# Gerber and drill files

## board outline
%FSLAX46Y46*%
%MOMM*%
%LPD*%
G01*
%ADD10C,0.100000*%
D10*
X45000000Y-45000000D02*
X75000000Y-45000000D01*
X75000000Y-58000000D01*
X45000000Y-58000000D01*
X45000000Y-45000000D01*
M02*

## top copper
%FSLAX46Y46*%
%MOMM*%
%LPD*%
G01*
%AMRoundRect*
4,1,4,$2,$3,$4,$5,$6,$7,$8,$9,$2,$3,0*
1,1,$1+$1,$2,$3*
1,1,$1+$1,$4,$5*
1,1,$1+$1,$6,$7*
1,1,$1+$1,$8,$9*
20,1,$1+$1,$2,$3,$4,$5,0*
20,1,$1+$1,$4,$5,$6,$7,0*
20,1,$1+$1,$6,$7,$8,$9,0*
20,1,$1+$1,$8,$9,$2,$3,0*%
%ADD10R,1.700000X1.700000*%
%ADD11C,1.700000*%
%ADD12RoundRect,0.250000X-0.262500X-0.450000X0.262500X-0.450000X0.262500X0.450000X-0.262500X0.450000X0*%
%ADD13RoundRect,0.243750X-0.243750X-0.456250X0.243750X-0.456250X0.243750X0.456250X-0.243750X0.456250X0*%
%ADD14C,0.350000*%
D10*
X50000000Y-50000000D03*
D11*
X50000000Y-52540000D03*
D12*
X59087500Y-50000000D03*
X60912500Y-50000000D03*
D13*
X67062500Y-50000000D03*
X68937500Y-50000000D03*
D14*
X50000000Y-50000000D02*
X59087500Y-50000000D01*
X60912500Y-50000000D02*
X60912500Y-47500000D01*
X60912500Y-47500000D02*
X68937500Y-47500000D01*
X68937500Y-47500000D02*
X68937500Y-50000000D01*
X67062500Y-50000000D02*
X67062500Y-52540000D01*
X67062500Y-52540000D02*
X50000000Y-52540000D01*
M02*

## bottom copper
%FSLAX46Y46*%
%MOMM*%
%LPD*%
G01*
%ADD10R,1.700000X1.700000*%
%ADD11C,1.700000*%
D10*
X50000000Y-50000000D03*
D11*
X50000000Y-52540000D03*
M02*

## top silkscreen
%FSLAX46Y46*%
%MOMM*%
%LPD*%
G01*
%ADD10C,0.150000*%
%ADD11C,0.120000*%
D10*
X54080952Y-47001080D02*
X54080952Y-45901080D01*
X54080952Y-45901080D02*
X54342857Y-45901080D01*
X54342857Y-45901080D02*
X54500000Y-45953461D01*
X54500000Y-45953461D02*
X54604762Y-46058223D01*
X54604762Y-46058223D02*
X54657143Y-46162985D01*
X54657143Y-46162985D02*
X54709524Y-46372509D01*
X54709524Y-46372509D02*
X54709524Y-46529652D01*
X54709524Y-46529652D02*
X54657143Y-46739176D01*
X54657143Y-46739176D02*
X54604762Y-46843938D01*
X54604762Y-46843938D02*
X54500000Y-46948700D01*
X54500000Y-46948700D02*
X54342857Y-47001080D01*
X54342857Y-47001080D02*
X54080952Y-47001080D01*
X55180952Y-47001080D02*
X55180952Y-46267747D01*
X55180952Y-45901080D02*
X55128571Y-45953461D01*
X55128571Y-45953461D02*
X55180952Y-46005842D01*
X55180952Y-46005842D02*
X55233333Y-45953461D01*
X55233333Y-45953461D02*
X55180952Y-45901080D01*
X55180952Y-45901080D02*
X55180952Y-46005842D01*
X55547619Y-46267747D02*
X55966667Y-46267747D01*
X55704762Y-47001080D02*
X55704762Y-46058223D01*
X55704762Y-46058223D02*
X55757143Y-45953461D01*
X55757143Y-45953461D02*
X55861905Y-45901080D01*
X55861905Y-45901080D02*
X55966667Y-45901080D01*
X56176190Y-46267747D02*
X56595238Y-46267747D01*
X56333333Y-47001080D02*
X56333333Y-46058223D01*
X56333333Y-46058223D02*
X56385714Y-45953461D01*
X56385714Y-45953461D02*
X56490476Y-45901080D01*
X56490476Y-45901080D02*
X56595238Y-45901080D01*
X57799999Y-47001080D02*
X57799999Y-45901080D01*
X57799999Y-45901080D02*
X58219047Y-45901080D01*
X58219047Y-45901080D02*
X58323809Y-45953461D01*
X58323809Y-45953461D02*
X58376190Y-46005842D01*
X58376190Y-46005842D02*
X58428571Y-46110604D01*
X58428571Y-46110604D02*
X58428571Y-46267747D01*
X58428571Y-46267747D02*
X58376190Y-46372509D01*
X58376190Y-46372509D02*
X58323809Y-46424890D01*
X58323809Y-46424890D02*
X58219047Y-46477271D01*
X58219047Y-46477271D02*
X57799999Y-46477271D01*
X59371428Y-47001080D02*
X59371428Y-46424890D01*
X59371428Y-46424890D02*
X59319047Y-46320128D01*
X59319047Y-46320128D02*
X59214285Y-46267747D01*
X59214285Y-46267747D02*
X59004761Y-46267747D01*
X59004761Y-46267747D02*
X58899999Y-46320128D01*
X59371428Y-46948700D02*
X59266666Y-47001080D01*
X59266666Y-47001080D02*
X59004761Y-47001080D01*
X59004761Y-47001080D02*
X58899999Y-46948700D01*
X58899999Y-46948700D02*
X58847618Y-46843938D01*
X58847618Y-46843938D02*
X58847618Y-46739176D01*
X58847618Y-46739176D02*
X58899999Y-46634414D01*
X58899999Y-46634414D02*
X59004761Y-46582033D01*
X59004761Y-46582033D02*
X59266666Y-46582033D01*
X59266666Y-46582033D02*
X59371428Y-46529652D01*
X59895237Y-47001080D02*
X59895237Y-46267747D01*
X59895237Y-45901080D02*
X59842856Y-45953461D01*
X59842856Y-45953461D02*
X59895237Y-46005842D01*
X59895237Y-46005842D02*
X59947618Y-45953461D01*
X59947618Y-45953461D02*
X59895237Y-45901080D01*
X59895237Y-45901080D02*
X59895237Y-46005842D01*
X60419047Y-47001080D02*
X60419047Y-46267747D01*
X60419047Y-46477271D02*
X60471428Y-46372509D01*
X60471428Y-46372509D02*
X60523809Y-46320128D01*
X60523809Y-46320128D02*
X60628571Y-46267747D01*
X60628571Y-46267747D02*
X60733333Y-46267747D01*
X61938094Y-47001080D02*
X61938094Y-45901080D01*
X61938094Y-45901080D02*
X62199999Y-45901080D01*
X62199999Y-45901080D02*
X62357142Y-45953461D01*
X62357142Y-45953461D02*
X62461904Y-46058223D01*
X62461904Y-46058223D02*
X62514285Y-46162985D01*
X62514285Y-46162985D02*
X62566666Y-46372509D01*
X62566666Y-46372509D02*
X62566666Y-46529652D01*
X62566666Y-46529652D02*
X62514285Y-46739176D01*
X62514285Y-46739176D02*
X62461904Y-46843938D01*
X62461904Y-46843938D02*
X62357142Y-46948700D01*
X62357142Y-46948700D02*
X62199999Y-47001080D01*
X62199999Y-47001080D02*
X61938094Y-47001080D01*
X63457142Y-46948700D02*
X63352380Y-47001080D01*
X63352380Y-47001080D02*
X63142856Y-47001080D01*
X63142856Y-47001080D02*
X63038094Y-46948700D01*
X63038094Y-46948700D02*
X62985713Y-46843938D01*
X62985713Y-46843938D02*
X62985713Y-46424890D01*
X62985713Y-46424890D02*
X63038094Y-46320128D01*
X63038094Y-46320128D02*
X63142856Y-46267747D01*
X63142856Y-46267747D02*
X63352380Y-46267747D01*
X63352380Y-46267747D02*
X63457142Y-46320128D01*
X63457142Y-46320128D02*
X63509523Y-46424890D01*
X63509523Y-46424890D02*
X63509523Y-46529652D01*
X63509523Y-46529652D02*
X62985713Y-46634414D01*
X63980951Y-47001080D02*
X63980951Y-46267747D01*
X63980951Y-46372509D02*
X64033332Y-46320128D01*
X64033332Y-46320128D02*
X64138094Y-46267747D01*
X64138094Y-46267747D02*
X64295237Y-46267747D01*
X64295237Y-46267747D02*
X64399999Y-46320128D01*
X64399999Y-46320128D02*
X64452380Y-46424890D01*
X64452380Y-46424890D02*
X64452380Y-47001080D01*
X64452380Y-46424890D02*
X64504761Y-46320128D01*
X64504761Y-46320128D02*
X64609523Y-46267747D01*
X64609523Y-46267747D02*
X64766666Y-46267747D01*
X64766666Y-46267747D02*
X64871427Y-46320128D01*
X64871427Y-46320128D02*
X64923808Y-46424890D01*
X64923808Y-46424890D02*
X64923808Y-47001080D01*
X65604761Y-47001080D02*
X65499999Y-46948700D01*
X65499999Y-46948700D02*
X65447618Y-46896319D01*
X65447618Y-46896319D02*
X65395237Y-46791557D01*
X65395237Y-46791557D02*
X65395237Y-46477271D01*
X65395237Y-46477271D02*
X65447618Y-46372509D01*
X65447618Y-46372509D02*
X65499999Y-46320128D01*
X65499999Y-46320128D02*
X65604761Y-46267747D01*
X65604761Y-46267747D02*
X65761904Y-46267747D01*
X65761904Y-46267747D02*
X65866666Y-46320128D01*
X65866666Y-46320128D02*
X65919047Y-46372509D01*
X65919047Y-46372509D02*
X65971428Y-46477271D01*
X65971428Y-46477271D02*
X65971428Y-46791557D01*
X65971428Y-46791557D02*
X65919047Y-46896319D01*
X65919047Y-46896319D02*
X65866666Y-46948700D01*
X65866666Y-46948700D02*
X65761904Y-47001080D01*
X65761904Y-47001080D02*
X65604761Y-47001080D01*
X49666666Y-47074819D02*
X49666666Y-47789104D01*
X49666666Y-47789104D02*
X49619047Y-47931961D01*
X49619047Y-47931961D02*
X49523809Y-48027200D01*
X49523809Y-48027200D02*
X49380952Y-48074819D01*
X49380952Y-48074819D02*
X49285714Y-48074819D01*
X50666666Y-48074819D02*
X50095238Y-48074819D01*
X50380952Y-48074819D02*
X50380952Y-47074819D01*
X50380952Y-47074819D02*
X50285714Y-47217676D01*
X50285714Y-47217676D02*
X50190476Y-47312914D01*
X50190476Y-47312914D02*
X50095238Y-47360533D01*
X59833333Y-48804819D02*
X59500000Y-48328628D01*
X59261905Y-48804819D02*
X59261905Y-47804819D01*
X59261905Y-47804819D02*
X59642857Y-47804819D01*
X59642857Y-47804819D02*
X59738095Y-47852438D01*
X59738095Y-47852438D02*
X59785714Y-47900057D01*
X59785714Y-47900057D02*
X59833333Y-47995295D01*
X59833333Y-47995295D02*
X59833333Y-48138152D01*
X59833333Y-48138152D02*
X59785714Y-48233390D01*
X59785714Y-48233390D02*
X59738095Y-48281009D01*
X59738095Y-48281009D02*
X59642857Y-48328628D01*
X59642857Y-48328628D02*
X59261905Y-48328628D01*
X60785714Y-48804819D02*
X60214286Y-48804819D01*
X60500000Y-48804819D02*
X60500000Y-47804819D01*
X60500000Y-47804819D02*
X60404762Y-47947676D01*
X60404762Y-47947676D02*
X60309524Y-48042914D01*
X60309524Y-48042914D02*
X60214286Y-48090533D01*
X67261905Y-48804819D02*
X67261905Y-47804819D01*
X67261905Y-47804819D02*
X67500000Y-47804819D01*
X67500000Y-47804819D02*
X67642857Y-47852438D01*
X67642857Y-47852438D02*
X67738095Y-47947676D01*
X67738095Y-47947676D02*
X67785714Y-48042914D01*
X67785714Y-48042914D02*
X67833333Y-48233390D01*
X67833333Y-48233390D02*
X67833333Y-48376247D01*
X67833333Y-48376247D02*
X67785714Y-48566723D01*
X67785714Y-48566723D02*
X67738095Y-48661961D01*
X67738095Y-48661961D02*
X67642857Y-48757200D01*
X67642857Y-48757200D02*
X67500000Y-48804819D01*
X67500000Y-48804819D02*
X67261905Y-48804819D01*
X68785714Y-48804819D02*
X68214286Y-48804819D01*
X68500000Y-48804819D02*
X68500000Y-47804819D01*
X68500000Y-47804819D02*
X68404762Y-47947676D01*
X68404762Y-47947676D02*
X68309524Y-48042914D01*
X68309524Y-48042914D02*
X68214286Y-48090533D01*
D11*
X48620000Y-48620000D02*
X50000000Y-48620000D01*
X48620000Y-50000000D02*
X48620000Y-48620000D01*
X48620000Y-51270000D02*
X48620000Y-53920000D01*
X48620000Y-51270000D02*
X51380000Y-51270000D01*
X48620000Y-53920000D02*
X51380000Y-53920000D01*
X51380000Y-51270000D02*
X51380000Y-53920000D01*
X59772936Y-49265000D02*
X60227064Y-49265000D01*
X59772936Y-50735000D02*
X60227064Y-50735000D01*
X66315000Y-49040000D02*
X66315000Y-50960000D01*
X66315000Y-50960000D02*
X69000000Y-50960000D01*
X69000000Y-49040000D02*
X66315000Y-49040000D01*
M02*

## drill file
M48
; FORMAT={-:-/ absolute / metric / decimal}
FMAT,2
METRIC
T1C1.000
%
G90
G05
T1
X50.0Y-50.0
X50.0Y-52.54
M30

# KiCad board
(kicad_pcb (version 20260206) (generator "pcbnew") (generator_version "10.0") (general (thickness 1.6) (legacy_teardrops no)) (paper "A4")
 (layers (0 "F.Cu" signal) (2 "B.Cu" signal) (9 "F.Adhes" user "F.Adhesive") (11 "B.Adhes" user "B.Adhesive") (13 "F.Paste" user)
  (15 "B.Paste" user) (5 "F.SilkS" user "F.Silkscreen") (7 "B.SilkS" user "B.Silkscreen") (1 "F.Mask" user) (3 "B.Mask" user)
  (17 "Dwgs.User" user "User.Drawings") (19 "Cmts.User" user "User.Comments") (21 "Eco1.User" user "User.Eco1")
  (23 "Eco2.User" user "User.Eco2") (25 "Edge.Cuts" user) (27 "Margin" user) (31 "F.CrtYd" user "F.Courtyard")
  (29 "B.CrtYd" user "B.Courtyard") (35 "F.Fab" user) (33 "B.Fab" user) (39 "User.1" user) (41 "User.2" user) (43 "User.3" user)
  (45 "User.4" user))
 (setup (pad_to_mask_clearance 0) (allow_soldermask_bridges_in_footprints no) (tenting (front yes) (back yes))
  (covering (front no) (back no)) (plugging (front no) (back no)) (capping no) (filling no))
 (gr_rect (start 45 45) (end 75 58) (stroke (width 0.1) (type solid)) (fill no) (layer "Edge.Cuts"))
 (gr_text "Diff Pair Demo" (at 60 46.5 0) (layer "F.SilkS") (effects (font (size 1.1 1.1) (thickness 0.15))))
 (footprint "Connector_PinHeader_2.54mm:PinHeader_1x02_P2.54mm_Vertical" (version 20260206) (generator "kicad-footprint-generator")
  (layer "F.Cu") (at 50 50 0)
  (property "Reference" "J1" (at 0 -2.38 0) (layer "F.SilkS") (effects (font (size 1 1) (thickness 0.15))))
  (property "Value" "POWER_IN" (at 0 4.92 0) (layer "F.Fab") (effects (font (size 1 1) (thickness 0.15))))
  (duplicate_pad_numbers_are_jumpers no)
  (fp_line (start -1.38 -1.38) (end 0 -1.38) (stroke (width 0.12) (type solid)) (layer "F.SilkS"))
  (fp_line (start -1.38 0) (end -1.38 -1.38) (stroke (width 0.12) (type solid)) (layer "F.SilkS"))
  (fp_line (start -1.38 1.27) (end -1.38 3.92) (stroke (width 0.12) (type solid)) (layer "F.SilkS"))
  (fp_line (start -1.38 1.27) (end 1.38 1.27) (stroke (width 0.12) (type solid)) (layer "F.SilkS"))
  (fp_line (start -1.38 3.92) (end 1.38 3.92) (stroke (width 0.12) (type solid)) (layer "F.SilkS"))
  (fp_line (start 1.38 1.27) (end 1.38 3.92) (stroke (width 0.12) (type solid)) (layer "F.SilkS"))
  (pad "1" thru_hole rect (at 0 0) (size 1.7 1.7) (drill 1) (layers "*.Cu" "*.Mask") (remove_unused_layers no) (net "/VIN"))
  (pad "2" thru_hole circle (at 0 2.54) (size 1.7 1.7) (drill 1) (layers "*.Cu" "*.Mask") (remove_unused_layers no) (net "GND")))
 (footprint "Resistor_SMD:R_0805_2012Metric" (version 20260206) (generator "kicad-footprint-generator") (layer "F.Cu") (at 60 50 0)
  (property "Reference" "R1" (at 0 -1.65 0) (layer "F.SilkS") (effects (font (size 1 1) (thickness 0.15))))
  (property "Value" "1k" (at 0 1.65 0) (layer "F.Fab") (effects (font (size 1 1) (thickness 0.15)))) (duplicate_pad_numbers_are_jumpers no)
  (fp_line (start -0.227064 -0.735) (end 0.227064 -0.735) (stroke (width 0.12) (type solid)) (layer "F.SilkS"))
  (fp_line (start -0.227064 0.735) (end 0.227064 0.735) (stroke (width 0.12) (type solid)) (layer "F.SilkS"))
  (pad "1" smd roundrect (at -0.9125 0) (size 1.025 1.4) (layers "F.Cu" "F.Mask" "F.Paste") (roundrect_rratio 0.243902) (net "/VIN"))
  (pad "2" smd roundrect (at 0.9125 0) (size 1.025 1.4) (layers "F.Cu" "F.Mask" "F.Paste") (roundrect_rratio 0.243902) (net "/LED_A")))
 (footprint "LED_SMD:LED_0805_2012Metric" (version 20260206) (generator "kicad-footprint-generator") (layer "F.Cu") (at 68 50 0)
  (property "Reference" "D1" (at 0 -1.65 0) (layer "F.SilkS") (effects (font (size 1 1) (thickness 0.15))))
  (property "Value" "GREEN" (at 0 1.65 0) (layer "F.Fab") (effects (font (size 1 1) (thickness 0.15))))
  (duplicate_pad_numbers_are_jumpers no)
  (fp_line (start -1.685 -0.96) (end -1.685 0.96) (stroke (width 0.12) (type solid)) (layer "F.SilkS"))
  (fp_line (start -1.685 0.96) (end 1 0.96) (stroke (width 0.12) (type solid)) (layer "F.SilkS"))
  (fp_line (start 1 -0.96) (end -1.685 -0.96) (stroke (width 0.12) (type solid)) (layer "F.SilkS"))
  (pad "1" smd roundrect (at -0.9375 0) (size 0.975 1.4) (layers "F.Cu" "F.Mask" "F.Paste") (roundrect_rratio 0.25) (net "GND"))
  (pad "2" smd roundrect (at 0.9375 0) (size 0.975 1.4) (layers "F.Cu" "F.Mask" "F.Paste") (roundrect_rratio 0.25) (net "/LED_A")))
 (segment (start 50 50) (end 59.0875 50) (width 0.35) (layer "F.Cu") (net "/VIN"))
 (segment (start 60.9125 50) (end 60.9125 47.5) (width 0.35) (layer "F.Cu") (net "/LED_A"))
 (segment (start 60.9125 47.5) (end 68.9375 47.5) (width 0.35) (layer "F.Cu") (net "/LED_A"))
 (segment (start 68.9375 47.5) (end 68.9375 50) (width 0.35) (layer "F.Cu") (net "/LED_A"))
 (segment (start 67.0625 50) (end 67.0625 52.54) (width 0.35) (layer "F.Cu") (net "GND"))
 (segment (start 67.0625 52.54) (end 50 52.54) (width 0.35) (layer "F.Cu") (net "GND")))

